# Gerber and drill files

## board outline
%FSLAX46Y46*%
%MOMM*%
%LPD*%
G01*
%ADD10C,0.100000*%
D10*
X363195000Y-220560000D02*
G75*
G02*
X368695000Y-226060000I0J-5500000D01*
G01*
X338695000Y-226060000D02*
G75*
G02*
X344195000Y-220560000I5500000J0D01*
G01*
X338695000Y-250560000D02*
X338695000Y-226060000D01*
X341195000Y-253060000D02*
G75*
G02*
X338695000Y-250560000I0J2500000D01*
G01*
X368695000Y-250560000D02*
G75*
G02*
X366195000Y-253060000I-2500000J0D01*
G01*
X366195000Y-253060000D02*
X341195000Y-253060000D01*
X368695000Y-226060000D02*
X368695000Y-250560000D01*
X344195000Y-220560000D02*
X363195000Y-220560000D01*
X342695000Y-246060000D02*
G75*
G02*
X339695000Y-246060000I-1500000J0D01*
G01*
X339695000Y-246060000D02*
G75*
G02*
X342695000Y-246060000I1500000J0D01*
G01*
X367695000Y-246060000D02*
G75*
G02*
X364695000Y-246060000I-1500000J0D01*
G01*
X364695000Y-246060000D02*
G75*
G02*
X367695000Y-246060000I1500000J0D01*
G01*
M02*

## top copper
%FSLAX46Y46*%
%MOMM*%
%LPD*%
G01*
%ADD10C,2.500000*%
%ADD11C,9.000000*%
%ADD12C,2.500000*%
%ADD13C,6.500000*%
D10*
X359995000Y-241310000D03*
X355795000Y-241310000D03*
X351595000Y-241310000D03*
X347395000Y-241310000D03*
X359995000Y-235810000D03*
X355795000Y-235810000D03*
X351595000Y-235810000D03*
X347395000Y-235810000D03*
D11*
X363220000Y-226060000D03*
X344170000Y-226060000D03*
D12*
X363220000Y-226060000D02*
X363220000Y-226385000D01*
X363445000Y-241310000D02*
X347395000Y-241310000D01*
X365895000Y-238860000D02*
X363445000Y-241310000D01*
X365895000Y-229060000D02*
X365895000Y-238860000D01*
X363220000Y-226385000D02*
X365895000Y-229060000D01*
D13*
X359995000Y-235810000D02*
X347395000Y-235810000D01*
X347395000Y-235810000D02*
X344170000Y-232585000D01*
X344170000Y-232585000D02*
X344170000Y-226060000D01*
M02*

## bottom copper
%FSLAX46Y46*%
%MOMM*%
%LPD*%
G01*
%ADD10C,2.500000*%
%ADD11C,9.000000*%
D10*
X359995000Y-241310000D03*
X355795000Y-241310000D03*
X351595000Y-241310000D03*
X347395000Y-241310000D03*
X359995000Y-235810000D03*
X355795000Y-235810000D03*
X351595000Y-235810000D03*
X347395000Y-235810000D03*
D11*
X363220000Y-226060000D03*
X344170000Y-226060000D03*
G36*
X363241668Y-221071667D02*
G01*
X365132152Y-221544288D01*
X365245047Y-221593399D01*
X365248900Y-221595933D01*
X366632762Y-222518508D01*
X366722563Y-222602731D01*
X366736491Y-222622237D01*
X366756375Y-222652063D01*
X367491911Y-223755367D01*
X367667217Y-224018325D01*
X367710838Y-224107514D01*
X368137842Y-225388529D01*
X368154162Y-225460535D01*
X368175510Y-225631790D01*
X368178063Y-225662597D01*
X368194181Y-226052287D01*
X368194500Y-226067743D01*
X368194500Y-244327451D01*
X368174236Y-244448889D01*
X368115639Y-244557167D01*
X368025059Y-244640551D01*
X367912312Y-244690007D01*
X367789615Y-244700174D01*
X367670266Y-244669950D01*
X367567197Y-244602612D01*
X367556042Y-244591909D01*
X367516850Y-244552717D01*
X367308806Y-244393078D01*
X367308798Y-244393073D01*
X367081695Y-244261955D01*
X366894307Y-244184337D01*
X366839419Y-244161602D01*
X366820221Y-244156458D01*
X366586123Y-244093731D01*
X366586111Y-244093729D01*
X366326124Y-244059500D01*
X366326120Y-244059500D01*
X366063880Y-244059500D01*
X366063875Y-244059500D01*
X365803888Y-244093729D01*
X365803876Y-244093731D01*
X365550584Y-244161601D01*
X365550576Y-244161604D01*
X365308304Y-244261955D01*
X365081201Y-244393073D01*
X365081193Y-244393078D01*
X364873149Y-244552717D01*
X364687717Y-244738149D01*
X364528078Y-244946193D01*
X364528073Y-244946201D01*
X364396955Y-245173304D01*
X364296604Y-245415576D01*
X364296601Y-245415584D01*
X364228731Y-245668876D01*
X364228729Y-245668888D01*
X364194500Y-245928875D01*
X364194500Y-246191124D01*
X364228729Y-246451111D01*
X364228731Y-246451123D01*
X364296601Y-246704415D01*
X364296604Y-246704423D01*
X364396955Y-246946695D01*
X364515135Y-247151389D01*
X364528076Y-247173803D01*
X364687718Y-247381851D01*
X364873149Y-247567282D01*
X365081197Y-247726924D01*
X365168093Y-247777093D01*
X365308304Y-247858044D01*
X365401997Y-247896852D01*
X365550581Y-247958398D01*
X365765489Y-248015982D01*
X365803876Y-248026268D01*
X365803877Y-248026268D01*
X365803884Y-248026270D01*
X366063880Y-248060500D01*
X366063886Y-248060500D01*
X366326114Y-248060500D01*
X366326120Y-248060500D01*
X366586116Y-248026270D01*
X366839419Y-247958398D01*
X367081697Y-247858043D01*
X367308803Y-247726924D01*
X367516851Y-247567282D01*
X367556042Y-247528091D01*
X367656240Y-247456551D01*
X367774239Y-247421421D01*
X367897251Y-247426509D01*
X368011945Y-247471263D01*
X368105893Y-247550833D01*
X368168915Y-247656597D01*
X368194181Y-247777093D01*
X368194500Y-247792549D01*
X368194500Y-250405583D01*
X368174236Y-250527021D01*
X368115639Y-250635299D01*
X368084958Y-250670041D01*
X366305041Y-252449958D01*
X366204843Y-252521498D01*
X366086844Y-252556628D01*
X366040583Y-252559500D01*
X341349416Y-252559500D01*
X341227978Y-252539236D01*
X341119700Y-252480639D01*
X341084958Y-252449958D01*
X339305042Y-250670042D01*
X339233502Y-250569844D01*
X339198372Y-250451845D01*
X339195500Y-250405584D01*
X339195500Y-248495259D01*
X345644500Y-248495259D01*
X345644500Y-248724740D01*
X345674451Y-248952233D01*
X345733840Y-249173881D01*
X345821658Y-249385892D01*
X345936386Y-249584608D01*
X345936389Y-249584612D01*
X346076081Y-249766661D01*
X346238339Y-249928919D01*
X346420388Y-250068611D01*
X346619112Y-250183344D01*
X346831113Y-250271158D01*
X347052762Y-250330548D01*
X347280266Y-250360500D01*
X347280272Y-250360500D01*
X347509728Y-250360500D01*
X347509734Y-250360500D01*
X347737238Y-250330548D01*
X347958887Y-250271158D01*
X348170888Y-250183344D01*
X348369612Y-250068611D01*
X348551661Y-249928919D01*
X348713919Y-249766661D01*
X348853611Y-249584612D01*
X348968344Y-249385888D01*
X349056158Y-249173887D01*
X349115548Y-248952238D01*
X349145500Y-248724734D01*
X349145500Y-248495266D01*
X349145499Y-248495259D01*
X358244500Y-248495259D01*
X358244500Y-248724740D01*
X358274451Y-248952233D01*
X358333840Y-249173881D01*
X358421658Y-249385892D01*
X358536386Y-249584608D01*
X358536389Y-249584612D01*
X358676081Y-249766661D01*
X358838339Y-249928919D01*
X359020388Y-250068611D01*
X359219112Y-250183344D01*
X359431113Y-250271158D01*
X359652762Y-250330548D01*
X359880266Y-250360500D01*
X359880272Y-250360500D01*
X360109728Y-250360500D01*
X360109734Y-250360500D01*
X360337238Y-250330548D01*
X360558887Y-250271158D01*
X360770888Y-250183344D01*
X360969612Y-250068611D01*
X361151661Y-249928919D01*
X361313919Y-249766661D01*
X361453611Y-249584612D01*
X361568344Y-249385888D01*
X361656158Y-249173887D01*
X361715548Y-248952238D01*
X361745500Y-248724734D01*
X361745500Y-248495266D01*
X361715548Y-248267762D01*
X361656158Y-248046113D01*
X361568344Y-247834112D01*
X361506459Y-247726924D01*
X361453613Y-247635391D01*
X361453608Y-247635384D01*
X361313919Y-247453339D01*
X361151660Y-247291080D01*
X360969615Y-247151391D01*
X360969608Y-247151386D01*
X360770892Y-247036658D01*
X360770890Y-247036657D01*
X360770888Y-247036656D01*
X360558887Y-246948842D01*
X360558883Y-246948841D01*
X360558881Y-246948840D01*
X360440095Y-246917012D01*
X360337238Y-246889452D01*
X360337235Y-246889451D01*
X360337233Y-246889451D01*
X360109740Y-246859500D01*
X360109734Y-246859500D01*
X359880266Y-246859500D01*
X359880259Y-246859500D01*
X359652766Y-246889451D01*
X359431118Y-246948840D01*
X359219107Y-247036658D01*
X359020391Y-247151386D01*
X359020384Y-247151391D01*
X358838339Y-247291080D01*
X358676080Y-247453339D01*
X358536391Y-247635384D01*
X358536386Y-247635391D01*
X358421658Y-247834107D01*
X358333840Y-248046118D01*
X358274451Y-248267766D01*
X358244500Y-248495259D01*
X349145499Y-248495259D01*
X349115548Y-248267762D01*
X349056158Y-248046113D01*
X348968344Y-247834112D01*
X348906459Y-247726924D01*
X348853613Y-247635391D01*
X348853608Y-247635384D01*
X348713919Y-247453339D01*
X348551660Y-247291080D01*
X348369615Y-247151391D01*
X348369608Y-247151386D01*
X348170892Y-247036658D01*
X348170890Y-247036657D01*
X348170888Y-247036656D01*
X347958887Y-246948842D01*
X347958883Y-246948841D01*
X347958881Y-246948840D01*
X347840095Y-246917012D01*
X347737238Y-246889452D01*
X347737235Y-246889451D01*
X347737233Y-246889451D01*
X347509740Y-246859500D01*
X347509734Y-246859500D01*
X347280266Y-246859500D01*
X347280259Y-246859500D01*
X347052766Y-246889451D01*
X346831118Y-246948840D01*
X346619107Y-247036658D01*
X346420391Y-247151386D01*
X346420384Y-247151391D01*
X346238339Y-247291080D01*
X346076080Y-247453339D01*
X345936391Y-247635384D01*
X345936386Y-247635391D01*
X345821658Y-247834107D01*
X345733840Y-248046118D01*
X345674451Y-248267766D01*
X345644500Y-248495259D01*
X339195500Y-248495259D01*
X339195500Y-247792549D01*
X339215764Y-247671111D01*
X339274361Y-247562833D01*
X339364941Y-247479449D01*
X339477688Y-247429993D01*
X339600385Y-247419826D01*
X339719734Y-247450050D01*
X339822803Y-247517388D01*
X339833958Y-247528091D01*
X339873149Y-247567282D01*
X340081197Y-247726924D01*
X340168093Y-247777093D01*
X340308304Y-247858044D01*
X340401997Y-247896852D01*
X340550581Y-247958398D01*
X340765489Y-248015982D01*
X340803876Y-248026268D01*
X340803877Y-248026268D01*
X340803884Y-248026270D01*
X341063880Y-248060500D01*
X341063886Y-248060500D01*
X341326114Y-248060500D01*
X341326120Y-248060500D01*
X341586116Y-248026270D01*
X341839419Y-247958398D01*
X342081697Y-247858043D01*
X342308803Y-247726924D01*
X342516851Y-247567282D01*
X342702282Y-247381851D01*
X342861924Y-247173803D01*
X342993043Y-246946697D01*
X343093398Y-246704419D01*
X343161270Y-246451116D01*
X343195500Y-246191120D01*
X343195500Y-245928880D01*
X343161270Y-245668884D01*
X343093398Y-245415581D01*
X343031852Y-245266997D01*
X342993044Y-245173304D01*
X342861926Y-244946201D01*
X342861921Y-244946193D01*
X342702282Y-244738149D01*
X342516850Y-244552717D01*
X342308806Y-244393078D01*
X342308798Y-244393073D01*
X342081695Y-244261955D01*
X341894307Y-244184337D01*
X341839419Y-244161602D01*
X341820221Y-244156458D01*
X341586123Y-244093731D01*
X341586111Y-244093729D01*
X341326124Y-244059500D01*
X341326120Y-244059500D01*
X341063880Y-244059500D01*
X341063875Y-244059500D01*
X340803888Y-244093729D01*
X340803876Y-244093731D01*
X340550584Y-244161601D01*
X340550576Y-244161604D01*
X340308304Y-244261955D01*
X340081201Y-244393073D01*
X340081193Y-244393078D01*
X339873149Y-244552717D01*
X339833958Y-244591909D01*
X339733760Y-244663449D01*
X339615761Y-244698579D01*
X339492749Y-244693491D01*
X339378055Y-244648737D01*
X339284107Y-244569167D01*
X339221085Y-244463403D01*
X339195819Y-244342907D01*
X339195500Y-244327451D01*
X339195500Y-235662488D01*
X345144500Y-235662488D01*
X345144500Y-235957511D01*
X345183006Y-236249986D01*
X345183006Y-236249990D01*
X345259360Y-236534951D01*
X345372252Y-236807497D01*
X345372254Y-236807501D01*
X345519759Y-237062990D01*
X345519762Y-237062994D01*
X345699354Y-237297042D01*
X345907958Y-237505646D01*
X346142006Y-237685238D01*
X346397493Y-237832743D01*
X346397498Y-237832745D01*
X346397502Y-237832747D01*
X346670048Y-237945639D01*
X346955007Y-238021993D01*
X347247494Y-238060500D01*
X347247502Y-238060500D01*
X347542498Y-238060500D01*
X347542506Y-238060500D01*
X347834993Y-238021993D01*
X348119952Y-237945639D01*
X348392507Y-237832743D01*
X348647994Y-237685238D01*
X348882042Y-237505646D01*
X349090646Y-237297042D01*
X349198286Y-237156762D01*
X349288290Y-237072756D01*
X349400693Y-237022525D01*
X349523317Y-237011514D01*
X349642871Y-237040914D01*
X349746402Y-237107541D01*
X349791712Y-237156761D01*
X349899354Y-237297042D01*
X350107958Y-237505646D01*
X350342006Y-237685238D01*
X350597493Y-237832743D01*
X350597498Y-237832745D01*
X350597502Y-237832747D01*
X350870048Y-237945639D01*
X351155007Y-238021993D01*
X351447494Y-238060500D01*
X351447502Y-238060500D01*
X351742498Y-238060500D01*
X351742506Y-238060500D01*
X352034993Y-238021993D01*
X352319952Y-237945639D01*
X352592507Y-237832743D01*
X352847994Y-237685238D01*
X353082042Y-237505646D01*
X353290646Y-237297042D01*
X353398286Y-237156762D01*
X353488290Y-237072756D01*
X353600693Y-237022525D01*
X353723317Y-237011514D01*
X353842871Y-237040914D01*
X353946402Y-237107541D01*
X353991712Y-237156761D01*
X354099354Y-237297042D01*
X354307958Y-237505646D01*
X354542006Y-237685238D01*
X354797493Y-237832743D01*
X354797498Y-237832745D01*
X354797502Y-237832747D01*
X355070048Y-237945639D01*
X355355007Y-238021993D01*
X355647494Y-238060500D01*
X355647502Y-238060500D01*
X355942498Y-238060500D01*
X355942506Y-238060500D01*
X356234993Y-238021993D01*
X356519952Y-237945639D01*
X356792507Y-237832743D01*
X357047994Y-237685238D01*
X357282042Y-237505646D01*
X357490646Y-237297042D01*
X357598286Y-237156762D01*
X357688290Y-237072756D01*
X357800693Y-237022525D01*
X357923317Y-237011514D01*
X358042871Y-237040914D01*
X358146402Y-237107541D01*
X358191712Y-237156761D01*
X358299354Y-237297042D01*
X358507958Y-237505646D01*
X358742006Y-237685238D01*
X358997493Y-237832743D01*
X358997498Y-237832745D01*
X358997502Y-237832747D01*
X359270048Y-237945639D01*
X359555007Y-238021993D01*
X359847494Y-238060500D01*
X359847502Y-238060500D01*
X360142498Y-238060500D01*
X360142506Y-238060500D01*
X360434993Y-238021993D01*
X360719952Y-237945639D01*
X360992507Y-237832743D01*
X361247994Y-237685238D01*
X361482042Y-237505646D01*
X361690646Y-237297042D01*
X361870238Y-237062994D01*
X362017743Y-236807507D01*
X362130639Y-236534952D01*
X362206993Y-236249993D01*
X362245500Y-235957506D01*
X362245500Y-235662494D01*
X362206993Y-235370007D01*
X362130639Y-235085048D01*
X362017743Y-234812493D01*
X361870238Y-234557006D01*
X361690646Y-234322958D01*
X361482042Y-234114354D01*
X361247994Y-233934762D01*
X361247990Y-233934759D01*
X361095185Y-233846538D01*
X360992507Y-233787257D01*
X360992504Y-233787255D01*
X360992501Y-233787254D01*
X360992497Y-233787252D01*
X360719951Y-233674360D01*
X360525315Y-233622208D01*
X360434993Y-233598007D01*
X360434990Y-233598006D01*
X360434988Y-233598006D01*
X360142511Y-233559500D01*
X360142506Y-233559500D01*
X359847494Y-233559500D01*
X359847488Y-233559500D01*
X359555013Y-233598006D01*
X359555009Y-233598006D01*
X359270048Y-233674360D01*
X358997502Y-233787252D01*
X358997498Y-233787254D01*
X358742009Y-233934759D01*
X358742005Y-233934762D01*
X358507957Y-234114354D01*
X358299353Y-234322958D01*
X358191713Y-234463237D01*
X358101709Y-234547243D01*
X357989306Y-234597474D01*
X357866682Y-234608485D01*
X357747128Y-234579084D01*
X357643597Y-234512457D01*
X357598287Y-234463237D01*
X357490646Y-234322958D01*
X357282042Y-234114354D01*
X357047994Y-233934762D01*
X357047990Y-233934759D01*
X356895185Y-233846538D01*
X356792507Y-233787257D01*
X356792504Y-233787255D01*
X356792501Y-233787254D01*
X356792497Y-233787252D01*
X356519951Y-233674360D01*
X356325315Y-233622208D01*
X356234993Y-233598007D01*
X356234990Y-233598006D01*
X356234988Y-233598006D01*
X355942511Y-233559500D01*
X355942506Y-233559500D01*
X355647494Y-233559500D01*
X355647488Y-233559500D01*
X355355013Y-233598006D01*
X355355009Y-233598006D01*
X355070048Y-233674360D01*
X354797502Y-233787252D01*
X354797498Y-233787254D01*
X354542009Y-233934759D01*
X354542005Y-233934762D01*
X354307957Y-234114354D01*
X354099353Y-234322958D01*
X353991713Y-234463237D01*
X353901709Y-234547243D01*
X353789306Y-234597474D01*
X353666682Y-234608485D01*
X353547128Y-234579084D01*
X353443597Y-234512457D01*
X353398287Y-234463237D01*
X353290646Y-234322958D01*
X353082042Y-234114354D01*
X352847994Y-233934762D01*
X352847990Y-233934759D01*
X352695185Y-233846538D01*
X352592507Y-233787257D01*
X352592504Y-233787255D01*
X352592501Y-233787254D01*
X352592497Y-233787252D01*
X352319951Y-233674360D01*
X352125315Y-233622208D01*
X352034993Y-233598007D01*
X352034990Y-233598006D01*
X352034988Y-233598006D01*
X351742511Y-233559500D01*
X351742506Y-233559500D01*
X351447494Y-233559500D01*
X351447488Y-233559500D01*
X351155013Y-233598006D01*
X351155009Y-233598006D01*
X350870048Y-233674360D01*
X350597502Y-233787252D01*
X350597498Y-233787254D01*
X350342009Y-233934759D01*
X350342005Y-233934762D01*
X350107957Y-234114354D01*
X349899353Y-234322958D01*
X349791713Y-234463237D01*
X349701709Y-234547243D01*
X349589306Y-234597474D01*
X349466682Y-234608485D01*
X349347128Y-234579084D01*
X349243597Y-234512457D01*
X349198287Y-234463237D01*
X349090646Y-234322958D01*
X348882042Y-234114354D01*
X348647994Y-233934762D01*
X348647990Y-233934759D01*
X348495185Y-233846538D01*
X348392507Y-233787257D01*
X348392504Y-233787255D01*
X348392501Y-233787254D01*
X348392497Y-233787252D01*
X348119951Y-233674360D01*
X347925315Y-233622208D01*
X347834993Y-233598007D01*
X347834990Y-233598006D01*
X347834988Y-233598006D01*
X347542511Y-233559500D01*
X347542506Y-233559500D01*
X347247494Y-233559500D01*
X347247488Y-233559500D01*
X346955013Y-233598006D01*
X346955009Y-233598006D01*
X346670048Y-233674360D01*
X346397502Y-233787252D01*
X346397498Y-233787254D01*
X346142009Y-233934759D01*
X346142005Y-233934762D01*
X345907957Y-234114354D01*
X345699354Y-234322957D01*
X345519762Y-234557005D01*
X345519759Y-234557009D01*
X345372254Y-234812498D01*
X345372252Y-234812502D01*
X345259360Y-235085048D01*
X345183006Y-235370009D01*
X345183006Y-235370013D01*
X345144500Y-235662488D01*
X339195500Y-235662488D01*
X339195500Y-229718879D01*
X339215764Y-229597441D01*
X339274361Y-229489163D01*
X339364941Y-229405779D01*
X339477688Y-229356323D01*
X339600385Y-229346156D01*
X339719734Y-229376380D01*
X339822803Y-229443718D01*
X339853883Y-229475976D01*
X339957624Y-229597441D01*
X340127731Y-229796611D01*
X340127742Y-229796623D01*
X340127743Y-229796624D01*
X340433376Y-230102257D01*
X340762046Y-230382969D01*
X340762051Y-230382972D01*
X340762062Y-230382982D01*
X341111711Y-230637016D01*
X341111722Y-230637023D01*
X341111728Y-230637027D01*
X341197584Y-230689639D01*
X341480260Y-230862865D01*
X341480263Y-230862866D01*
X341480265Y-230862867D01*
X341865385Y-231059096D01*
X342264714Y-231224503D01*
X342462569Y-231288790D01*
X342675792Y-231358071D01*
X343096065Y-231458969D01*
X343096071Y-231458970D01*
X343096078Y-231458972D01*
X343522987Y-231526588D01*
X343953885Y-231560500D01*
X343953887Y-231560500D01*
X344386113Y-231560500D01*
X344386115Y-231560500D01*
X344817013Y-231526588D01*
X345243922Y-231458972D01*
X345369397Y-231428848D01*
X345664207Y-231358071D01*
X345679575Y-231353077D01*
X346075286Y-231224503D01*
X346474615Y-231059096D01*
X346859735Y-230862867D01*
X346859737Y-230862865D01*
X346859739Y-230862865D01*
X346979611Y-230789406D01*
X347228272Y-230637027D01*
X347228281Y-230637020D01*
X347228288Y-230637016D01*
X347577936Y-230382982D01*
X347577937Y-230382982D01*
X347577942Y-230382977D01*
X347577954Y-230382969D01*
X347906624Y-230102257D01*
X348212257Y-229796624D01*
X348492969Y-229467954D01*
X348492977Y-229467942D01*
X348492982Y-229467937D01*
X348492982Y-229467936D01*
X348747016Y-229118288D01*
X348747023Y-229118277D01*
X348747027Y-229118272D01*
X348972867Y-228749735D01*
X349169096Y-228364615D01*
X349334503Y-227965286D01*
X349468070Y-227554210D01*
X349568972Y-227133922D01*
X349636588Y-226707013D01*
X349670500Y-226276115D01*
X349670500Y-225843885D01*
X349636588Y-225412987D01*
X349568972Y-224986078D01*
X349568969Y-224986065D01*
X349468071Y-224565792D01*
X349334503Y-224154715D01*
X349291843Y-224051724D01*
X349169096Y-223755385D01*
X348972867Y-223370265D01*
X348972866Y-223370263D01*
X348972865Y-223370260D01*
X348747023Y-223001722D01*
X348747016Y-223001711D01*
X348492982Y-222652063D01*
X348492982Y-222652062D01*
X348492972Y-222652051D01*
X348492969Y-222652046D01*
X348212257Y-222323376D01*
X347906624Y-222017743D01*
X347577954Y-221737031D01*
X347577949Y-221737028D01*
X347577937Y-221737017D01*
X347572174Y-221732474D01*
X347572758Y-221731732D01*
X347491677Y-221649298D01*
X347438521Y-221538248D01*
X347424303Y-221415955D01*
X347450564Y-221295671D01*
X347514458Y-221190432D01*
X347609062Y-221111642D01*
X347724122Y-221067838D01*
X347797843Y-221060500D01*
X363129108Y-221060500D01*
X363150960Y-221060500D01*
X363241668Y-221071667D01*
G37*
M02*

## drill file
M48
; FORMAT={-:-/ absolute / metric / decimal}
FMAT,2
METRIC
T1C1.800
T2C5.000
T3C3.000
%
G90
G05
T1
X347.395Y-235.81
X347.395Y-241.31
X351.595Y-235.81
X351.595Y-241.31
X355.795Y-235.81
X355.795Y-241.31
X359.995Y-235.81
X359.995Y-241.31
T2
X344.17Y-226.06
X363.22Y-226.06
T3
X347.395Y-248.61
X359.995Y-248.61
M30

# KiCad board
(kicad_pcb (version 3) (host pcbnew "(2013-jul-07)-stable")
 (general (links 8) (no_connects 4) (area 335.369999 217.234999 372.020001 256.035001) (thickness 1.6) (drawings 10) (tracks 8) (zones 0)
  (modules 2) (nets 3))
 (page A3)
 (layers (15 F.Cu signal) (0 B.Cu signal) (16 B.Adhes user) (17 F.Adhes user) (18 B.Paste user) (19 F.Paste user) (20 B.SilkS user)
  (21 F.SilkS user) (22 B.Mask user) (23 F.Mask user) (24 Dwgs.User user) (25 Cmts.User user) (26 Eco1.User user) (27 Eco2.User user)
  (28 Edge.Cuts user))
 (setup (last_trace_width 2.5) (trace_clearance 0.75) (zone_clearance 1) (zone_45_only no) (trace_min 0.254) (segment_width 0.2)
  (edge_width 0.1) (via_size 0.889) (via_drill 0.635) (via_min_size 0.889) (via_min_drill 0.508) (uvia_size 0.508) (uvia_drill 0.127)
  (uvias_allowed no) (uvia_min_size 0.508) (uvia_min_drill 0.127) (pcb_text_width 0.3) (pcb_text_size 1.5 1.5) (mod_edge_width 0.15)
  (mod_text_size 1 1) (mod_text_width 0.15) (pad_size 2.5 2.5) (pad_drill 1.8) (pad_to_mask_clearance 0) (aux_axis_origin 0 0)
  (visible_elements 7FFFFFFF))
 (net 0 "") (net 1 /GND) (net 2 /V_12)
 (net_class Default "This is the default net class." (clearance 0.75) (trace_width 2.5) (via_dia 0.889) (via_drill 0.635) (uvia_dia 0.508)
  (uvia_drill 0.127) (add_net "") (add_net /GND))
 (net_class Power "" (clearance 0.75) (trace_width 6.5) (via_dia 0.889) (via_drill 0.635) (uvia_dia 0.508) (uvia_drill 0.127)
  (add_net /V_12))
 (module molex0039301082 (layer F.Cu) (at 353.695 238.56)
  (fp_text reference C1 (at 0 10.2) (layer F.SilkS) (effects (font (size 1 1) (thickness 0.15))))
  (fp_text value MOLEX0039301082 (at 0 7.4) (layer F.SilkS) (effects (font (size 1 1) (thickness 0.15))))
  (pad 1 thru_hole circle (at 6.3 2.75) (size 2.5 2.5) (drill 1.8) (layers *.Cu *.Mask F.SilkS) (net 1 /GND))
  (pad 2 thru_hole circle (at 2.1 2.75) (size 2.5 2.5) (drill 1.8) (layers *.Cu *.Mask F.SilkS) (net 1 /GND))
  (pad 3 thru_hole circle (at -2.1 2.75) (size 2.5 2.5) (drill 1.8) (layers *.Cu *.Mask F.SilkS) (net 1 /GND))
  (pad 4 thru_hole circle (at -6.3 2.75) (size 2.5 2.5) (drill 1.8) (layers *.Cu *.Mask F.SilkS) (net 1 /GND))
  (pad 5 thru_hole circle (at 6.3 -2.75) (size 2.5 2.5) (drill 1.8) (layers *.Cu *.Mask F.SilkS) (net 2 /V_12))
  (pad 6 thru_hole circle (at 2.1 -2.75) (size 2.5 2.5) (drill 1.8) (layers *.Cu *.Mask F.SilkS) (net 2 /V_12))
  (pad 7 thru_hole circle (at -2.1 -2.75) (size 2.5 2.5) (drill 1.8) (layers *.Cu *.Mask F.SilkS) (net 2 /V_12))
  (pad 8 thru_hole circle (at -6.3 -2.75) (size 2.5 2.5) (drill 1.8) (layers *.Cu *.Mask F.SilkS) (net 2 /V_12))
  (pad "" np_thru_hole circle (at 6.3 10.05) (size 3 3) (drill 3) (layers *.Cu *.Mask F.SilkS))
  (pad "" np_thru_hole circle (at -6.3 10.05) (size 3 3) (drill 3) (layers *.Cu *.Mask F.SilkS)))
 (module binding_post (layer F.Cu) (at 353.695 226.06)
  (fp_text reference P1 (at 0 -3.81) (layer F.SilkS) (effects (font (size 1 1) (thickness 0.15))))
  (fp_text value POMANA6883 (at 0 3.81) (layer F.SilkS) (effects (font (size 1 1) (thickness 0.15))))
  (pad 1 thru_hole circle (at 9.525 0) (size 9 9) (drill 5) (layers *.Cu *.Mask F.SilkS) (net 1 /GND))
  (pad 2 thru_hole circle (at -9.525 0) (size 9 9) (drill 5) (layers *.Cu *.Mask F.SilkS) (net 2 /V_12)))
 (gr_arc (start 363.195 226.06) (end 363.195 220.56) (angle 90) (layer Edge.Cuts) (width 0.1))
 (gr_arc (start 344.195 226.06) (end 338.695 226.06) (angle 90) (layer Edge.Cuts) (width 0.1))
 (gr_line (start 338.695 250.56) (end 338.695 226.06) (angle 90) (layer Edge.Cuts) (width 0.1))
 (gr_arc (start 341.195 250.56) (end 341.195 253.06) (angle 90) (layer Edge.Cuts) (width 0.1))
 (gr_arc (start 366.195 250.56) (end 368.695 250.56) (angle 90) (layer Edge.Cuts) (width 0.1))
 (gr_line (start 366.195 253.06) (end 341.195 253.06) (angle 90) (layer Edge.Cuts) (width 0.1))
 (gr_line (start 368.695 226.06) (end 368.695 250.56) (angle 90) (layer Edge.Cuts) (width 0.1))
 (gr_line (start 344.195 220.56) (end 363.195 220.56) (angle 90) (layer Edge.Cuts) (width 0.1))
 (gr_circle (center 341.195 246.06) (end 341.195 247.56) (layer Edge.Cuts) (width 0.1))
 (gr_circle (center 366.195 246.06) (end 367.695 246.06) (layer Edge.Cuts) (width 0.1))
 (segment (start 363.22 226.06) (end 363.22 226.385) (width 2.5) (layer F.Cu) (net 1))
 (segment (start 363.445 241.31) (end 347.395 241.31) (width 2.5) (layer F.Cu) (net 1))
 (segment (start 365.895 238.86) (end 363.445 241.31) (width 2.5) (layer F.Cu) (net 1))
 (segment (start 365.895 229.06) (end 365.895 238.86) (width 2.5) (layer F.Cu) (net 1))
 (segment (start 363.22 226.385) (end 365.895 229.06) (width 2.5) (layer F.Cu) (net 1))
 (segment (start 359.995 235.81) (end 347.395 235.81) (width 6.5) (layer F.Cu) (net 2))
 (segment (start 347.395 235.81) (end 344.17 232.585) (width 6.5) (layer F.Cu) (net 2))
 (segment (start 344.17 232.585) (end 344.17 226.06) (width 6.5) (layer F.Cu) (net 2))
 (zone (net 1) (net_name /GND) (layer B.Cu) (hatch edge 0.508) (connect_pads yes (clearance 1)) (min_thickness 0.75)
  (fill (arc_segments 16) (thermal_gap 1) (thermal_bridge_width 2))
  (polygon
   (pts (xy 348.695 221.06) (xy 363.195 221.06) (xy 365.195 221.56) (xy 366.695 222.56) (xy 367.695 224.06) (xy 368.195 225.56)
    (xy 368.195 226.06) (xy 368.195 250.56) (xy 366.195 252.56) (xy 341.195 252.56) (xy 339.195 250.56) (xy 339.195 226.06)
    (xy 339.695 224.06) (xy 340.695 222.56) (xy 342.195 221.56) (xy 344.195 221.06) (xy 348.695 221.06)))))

